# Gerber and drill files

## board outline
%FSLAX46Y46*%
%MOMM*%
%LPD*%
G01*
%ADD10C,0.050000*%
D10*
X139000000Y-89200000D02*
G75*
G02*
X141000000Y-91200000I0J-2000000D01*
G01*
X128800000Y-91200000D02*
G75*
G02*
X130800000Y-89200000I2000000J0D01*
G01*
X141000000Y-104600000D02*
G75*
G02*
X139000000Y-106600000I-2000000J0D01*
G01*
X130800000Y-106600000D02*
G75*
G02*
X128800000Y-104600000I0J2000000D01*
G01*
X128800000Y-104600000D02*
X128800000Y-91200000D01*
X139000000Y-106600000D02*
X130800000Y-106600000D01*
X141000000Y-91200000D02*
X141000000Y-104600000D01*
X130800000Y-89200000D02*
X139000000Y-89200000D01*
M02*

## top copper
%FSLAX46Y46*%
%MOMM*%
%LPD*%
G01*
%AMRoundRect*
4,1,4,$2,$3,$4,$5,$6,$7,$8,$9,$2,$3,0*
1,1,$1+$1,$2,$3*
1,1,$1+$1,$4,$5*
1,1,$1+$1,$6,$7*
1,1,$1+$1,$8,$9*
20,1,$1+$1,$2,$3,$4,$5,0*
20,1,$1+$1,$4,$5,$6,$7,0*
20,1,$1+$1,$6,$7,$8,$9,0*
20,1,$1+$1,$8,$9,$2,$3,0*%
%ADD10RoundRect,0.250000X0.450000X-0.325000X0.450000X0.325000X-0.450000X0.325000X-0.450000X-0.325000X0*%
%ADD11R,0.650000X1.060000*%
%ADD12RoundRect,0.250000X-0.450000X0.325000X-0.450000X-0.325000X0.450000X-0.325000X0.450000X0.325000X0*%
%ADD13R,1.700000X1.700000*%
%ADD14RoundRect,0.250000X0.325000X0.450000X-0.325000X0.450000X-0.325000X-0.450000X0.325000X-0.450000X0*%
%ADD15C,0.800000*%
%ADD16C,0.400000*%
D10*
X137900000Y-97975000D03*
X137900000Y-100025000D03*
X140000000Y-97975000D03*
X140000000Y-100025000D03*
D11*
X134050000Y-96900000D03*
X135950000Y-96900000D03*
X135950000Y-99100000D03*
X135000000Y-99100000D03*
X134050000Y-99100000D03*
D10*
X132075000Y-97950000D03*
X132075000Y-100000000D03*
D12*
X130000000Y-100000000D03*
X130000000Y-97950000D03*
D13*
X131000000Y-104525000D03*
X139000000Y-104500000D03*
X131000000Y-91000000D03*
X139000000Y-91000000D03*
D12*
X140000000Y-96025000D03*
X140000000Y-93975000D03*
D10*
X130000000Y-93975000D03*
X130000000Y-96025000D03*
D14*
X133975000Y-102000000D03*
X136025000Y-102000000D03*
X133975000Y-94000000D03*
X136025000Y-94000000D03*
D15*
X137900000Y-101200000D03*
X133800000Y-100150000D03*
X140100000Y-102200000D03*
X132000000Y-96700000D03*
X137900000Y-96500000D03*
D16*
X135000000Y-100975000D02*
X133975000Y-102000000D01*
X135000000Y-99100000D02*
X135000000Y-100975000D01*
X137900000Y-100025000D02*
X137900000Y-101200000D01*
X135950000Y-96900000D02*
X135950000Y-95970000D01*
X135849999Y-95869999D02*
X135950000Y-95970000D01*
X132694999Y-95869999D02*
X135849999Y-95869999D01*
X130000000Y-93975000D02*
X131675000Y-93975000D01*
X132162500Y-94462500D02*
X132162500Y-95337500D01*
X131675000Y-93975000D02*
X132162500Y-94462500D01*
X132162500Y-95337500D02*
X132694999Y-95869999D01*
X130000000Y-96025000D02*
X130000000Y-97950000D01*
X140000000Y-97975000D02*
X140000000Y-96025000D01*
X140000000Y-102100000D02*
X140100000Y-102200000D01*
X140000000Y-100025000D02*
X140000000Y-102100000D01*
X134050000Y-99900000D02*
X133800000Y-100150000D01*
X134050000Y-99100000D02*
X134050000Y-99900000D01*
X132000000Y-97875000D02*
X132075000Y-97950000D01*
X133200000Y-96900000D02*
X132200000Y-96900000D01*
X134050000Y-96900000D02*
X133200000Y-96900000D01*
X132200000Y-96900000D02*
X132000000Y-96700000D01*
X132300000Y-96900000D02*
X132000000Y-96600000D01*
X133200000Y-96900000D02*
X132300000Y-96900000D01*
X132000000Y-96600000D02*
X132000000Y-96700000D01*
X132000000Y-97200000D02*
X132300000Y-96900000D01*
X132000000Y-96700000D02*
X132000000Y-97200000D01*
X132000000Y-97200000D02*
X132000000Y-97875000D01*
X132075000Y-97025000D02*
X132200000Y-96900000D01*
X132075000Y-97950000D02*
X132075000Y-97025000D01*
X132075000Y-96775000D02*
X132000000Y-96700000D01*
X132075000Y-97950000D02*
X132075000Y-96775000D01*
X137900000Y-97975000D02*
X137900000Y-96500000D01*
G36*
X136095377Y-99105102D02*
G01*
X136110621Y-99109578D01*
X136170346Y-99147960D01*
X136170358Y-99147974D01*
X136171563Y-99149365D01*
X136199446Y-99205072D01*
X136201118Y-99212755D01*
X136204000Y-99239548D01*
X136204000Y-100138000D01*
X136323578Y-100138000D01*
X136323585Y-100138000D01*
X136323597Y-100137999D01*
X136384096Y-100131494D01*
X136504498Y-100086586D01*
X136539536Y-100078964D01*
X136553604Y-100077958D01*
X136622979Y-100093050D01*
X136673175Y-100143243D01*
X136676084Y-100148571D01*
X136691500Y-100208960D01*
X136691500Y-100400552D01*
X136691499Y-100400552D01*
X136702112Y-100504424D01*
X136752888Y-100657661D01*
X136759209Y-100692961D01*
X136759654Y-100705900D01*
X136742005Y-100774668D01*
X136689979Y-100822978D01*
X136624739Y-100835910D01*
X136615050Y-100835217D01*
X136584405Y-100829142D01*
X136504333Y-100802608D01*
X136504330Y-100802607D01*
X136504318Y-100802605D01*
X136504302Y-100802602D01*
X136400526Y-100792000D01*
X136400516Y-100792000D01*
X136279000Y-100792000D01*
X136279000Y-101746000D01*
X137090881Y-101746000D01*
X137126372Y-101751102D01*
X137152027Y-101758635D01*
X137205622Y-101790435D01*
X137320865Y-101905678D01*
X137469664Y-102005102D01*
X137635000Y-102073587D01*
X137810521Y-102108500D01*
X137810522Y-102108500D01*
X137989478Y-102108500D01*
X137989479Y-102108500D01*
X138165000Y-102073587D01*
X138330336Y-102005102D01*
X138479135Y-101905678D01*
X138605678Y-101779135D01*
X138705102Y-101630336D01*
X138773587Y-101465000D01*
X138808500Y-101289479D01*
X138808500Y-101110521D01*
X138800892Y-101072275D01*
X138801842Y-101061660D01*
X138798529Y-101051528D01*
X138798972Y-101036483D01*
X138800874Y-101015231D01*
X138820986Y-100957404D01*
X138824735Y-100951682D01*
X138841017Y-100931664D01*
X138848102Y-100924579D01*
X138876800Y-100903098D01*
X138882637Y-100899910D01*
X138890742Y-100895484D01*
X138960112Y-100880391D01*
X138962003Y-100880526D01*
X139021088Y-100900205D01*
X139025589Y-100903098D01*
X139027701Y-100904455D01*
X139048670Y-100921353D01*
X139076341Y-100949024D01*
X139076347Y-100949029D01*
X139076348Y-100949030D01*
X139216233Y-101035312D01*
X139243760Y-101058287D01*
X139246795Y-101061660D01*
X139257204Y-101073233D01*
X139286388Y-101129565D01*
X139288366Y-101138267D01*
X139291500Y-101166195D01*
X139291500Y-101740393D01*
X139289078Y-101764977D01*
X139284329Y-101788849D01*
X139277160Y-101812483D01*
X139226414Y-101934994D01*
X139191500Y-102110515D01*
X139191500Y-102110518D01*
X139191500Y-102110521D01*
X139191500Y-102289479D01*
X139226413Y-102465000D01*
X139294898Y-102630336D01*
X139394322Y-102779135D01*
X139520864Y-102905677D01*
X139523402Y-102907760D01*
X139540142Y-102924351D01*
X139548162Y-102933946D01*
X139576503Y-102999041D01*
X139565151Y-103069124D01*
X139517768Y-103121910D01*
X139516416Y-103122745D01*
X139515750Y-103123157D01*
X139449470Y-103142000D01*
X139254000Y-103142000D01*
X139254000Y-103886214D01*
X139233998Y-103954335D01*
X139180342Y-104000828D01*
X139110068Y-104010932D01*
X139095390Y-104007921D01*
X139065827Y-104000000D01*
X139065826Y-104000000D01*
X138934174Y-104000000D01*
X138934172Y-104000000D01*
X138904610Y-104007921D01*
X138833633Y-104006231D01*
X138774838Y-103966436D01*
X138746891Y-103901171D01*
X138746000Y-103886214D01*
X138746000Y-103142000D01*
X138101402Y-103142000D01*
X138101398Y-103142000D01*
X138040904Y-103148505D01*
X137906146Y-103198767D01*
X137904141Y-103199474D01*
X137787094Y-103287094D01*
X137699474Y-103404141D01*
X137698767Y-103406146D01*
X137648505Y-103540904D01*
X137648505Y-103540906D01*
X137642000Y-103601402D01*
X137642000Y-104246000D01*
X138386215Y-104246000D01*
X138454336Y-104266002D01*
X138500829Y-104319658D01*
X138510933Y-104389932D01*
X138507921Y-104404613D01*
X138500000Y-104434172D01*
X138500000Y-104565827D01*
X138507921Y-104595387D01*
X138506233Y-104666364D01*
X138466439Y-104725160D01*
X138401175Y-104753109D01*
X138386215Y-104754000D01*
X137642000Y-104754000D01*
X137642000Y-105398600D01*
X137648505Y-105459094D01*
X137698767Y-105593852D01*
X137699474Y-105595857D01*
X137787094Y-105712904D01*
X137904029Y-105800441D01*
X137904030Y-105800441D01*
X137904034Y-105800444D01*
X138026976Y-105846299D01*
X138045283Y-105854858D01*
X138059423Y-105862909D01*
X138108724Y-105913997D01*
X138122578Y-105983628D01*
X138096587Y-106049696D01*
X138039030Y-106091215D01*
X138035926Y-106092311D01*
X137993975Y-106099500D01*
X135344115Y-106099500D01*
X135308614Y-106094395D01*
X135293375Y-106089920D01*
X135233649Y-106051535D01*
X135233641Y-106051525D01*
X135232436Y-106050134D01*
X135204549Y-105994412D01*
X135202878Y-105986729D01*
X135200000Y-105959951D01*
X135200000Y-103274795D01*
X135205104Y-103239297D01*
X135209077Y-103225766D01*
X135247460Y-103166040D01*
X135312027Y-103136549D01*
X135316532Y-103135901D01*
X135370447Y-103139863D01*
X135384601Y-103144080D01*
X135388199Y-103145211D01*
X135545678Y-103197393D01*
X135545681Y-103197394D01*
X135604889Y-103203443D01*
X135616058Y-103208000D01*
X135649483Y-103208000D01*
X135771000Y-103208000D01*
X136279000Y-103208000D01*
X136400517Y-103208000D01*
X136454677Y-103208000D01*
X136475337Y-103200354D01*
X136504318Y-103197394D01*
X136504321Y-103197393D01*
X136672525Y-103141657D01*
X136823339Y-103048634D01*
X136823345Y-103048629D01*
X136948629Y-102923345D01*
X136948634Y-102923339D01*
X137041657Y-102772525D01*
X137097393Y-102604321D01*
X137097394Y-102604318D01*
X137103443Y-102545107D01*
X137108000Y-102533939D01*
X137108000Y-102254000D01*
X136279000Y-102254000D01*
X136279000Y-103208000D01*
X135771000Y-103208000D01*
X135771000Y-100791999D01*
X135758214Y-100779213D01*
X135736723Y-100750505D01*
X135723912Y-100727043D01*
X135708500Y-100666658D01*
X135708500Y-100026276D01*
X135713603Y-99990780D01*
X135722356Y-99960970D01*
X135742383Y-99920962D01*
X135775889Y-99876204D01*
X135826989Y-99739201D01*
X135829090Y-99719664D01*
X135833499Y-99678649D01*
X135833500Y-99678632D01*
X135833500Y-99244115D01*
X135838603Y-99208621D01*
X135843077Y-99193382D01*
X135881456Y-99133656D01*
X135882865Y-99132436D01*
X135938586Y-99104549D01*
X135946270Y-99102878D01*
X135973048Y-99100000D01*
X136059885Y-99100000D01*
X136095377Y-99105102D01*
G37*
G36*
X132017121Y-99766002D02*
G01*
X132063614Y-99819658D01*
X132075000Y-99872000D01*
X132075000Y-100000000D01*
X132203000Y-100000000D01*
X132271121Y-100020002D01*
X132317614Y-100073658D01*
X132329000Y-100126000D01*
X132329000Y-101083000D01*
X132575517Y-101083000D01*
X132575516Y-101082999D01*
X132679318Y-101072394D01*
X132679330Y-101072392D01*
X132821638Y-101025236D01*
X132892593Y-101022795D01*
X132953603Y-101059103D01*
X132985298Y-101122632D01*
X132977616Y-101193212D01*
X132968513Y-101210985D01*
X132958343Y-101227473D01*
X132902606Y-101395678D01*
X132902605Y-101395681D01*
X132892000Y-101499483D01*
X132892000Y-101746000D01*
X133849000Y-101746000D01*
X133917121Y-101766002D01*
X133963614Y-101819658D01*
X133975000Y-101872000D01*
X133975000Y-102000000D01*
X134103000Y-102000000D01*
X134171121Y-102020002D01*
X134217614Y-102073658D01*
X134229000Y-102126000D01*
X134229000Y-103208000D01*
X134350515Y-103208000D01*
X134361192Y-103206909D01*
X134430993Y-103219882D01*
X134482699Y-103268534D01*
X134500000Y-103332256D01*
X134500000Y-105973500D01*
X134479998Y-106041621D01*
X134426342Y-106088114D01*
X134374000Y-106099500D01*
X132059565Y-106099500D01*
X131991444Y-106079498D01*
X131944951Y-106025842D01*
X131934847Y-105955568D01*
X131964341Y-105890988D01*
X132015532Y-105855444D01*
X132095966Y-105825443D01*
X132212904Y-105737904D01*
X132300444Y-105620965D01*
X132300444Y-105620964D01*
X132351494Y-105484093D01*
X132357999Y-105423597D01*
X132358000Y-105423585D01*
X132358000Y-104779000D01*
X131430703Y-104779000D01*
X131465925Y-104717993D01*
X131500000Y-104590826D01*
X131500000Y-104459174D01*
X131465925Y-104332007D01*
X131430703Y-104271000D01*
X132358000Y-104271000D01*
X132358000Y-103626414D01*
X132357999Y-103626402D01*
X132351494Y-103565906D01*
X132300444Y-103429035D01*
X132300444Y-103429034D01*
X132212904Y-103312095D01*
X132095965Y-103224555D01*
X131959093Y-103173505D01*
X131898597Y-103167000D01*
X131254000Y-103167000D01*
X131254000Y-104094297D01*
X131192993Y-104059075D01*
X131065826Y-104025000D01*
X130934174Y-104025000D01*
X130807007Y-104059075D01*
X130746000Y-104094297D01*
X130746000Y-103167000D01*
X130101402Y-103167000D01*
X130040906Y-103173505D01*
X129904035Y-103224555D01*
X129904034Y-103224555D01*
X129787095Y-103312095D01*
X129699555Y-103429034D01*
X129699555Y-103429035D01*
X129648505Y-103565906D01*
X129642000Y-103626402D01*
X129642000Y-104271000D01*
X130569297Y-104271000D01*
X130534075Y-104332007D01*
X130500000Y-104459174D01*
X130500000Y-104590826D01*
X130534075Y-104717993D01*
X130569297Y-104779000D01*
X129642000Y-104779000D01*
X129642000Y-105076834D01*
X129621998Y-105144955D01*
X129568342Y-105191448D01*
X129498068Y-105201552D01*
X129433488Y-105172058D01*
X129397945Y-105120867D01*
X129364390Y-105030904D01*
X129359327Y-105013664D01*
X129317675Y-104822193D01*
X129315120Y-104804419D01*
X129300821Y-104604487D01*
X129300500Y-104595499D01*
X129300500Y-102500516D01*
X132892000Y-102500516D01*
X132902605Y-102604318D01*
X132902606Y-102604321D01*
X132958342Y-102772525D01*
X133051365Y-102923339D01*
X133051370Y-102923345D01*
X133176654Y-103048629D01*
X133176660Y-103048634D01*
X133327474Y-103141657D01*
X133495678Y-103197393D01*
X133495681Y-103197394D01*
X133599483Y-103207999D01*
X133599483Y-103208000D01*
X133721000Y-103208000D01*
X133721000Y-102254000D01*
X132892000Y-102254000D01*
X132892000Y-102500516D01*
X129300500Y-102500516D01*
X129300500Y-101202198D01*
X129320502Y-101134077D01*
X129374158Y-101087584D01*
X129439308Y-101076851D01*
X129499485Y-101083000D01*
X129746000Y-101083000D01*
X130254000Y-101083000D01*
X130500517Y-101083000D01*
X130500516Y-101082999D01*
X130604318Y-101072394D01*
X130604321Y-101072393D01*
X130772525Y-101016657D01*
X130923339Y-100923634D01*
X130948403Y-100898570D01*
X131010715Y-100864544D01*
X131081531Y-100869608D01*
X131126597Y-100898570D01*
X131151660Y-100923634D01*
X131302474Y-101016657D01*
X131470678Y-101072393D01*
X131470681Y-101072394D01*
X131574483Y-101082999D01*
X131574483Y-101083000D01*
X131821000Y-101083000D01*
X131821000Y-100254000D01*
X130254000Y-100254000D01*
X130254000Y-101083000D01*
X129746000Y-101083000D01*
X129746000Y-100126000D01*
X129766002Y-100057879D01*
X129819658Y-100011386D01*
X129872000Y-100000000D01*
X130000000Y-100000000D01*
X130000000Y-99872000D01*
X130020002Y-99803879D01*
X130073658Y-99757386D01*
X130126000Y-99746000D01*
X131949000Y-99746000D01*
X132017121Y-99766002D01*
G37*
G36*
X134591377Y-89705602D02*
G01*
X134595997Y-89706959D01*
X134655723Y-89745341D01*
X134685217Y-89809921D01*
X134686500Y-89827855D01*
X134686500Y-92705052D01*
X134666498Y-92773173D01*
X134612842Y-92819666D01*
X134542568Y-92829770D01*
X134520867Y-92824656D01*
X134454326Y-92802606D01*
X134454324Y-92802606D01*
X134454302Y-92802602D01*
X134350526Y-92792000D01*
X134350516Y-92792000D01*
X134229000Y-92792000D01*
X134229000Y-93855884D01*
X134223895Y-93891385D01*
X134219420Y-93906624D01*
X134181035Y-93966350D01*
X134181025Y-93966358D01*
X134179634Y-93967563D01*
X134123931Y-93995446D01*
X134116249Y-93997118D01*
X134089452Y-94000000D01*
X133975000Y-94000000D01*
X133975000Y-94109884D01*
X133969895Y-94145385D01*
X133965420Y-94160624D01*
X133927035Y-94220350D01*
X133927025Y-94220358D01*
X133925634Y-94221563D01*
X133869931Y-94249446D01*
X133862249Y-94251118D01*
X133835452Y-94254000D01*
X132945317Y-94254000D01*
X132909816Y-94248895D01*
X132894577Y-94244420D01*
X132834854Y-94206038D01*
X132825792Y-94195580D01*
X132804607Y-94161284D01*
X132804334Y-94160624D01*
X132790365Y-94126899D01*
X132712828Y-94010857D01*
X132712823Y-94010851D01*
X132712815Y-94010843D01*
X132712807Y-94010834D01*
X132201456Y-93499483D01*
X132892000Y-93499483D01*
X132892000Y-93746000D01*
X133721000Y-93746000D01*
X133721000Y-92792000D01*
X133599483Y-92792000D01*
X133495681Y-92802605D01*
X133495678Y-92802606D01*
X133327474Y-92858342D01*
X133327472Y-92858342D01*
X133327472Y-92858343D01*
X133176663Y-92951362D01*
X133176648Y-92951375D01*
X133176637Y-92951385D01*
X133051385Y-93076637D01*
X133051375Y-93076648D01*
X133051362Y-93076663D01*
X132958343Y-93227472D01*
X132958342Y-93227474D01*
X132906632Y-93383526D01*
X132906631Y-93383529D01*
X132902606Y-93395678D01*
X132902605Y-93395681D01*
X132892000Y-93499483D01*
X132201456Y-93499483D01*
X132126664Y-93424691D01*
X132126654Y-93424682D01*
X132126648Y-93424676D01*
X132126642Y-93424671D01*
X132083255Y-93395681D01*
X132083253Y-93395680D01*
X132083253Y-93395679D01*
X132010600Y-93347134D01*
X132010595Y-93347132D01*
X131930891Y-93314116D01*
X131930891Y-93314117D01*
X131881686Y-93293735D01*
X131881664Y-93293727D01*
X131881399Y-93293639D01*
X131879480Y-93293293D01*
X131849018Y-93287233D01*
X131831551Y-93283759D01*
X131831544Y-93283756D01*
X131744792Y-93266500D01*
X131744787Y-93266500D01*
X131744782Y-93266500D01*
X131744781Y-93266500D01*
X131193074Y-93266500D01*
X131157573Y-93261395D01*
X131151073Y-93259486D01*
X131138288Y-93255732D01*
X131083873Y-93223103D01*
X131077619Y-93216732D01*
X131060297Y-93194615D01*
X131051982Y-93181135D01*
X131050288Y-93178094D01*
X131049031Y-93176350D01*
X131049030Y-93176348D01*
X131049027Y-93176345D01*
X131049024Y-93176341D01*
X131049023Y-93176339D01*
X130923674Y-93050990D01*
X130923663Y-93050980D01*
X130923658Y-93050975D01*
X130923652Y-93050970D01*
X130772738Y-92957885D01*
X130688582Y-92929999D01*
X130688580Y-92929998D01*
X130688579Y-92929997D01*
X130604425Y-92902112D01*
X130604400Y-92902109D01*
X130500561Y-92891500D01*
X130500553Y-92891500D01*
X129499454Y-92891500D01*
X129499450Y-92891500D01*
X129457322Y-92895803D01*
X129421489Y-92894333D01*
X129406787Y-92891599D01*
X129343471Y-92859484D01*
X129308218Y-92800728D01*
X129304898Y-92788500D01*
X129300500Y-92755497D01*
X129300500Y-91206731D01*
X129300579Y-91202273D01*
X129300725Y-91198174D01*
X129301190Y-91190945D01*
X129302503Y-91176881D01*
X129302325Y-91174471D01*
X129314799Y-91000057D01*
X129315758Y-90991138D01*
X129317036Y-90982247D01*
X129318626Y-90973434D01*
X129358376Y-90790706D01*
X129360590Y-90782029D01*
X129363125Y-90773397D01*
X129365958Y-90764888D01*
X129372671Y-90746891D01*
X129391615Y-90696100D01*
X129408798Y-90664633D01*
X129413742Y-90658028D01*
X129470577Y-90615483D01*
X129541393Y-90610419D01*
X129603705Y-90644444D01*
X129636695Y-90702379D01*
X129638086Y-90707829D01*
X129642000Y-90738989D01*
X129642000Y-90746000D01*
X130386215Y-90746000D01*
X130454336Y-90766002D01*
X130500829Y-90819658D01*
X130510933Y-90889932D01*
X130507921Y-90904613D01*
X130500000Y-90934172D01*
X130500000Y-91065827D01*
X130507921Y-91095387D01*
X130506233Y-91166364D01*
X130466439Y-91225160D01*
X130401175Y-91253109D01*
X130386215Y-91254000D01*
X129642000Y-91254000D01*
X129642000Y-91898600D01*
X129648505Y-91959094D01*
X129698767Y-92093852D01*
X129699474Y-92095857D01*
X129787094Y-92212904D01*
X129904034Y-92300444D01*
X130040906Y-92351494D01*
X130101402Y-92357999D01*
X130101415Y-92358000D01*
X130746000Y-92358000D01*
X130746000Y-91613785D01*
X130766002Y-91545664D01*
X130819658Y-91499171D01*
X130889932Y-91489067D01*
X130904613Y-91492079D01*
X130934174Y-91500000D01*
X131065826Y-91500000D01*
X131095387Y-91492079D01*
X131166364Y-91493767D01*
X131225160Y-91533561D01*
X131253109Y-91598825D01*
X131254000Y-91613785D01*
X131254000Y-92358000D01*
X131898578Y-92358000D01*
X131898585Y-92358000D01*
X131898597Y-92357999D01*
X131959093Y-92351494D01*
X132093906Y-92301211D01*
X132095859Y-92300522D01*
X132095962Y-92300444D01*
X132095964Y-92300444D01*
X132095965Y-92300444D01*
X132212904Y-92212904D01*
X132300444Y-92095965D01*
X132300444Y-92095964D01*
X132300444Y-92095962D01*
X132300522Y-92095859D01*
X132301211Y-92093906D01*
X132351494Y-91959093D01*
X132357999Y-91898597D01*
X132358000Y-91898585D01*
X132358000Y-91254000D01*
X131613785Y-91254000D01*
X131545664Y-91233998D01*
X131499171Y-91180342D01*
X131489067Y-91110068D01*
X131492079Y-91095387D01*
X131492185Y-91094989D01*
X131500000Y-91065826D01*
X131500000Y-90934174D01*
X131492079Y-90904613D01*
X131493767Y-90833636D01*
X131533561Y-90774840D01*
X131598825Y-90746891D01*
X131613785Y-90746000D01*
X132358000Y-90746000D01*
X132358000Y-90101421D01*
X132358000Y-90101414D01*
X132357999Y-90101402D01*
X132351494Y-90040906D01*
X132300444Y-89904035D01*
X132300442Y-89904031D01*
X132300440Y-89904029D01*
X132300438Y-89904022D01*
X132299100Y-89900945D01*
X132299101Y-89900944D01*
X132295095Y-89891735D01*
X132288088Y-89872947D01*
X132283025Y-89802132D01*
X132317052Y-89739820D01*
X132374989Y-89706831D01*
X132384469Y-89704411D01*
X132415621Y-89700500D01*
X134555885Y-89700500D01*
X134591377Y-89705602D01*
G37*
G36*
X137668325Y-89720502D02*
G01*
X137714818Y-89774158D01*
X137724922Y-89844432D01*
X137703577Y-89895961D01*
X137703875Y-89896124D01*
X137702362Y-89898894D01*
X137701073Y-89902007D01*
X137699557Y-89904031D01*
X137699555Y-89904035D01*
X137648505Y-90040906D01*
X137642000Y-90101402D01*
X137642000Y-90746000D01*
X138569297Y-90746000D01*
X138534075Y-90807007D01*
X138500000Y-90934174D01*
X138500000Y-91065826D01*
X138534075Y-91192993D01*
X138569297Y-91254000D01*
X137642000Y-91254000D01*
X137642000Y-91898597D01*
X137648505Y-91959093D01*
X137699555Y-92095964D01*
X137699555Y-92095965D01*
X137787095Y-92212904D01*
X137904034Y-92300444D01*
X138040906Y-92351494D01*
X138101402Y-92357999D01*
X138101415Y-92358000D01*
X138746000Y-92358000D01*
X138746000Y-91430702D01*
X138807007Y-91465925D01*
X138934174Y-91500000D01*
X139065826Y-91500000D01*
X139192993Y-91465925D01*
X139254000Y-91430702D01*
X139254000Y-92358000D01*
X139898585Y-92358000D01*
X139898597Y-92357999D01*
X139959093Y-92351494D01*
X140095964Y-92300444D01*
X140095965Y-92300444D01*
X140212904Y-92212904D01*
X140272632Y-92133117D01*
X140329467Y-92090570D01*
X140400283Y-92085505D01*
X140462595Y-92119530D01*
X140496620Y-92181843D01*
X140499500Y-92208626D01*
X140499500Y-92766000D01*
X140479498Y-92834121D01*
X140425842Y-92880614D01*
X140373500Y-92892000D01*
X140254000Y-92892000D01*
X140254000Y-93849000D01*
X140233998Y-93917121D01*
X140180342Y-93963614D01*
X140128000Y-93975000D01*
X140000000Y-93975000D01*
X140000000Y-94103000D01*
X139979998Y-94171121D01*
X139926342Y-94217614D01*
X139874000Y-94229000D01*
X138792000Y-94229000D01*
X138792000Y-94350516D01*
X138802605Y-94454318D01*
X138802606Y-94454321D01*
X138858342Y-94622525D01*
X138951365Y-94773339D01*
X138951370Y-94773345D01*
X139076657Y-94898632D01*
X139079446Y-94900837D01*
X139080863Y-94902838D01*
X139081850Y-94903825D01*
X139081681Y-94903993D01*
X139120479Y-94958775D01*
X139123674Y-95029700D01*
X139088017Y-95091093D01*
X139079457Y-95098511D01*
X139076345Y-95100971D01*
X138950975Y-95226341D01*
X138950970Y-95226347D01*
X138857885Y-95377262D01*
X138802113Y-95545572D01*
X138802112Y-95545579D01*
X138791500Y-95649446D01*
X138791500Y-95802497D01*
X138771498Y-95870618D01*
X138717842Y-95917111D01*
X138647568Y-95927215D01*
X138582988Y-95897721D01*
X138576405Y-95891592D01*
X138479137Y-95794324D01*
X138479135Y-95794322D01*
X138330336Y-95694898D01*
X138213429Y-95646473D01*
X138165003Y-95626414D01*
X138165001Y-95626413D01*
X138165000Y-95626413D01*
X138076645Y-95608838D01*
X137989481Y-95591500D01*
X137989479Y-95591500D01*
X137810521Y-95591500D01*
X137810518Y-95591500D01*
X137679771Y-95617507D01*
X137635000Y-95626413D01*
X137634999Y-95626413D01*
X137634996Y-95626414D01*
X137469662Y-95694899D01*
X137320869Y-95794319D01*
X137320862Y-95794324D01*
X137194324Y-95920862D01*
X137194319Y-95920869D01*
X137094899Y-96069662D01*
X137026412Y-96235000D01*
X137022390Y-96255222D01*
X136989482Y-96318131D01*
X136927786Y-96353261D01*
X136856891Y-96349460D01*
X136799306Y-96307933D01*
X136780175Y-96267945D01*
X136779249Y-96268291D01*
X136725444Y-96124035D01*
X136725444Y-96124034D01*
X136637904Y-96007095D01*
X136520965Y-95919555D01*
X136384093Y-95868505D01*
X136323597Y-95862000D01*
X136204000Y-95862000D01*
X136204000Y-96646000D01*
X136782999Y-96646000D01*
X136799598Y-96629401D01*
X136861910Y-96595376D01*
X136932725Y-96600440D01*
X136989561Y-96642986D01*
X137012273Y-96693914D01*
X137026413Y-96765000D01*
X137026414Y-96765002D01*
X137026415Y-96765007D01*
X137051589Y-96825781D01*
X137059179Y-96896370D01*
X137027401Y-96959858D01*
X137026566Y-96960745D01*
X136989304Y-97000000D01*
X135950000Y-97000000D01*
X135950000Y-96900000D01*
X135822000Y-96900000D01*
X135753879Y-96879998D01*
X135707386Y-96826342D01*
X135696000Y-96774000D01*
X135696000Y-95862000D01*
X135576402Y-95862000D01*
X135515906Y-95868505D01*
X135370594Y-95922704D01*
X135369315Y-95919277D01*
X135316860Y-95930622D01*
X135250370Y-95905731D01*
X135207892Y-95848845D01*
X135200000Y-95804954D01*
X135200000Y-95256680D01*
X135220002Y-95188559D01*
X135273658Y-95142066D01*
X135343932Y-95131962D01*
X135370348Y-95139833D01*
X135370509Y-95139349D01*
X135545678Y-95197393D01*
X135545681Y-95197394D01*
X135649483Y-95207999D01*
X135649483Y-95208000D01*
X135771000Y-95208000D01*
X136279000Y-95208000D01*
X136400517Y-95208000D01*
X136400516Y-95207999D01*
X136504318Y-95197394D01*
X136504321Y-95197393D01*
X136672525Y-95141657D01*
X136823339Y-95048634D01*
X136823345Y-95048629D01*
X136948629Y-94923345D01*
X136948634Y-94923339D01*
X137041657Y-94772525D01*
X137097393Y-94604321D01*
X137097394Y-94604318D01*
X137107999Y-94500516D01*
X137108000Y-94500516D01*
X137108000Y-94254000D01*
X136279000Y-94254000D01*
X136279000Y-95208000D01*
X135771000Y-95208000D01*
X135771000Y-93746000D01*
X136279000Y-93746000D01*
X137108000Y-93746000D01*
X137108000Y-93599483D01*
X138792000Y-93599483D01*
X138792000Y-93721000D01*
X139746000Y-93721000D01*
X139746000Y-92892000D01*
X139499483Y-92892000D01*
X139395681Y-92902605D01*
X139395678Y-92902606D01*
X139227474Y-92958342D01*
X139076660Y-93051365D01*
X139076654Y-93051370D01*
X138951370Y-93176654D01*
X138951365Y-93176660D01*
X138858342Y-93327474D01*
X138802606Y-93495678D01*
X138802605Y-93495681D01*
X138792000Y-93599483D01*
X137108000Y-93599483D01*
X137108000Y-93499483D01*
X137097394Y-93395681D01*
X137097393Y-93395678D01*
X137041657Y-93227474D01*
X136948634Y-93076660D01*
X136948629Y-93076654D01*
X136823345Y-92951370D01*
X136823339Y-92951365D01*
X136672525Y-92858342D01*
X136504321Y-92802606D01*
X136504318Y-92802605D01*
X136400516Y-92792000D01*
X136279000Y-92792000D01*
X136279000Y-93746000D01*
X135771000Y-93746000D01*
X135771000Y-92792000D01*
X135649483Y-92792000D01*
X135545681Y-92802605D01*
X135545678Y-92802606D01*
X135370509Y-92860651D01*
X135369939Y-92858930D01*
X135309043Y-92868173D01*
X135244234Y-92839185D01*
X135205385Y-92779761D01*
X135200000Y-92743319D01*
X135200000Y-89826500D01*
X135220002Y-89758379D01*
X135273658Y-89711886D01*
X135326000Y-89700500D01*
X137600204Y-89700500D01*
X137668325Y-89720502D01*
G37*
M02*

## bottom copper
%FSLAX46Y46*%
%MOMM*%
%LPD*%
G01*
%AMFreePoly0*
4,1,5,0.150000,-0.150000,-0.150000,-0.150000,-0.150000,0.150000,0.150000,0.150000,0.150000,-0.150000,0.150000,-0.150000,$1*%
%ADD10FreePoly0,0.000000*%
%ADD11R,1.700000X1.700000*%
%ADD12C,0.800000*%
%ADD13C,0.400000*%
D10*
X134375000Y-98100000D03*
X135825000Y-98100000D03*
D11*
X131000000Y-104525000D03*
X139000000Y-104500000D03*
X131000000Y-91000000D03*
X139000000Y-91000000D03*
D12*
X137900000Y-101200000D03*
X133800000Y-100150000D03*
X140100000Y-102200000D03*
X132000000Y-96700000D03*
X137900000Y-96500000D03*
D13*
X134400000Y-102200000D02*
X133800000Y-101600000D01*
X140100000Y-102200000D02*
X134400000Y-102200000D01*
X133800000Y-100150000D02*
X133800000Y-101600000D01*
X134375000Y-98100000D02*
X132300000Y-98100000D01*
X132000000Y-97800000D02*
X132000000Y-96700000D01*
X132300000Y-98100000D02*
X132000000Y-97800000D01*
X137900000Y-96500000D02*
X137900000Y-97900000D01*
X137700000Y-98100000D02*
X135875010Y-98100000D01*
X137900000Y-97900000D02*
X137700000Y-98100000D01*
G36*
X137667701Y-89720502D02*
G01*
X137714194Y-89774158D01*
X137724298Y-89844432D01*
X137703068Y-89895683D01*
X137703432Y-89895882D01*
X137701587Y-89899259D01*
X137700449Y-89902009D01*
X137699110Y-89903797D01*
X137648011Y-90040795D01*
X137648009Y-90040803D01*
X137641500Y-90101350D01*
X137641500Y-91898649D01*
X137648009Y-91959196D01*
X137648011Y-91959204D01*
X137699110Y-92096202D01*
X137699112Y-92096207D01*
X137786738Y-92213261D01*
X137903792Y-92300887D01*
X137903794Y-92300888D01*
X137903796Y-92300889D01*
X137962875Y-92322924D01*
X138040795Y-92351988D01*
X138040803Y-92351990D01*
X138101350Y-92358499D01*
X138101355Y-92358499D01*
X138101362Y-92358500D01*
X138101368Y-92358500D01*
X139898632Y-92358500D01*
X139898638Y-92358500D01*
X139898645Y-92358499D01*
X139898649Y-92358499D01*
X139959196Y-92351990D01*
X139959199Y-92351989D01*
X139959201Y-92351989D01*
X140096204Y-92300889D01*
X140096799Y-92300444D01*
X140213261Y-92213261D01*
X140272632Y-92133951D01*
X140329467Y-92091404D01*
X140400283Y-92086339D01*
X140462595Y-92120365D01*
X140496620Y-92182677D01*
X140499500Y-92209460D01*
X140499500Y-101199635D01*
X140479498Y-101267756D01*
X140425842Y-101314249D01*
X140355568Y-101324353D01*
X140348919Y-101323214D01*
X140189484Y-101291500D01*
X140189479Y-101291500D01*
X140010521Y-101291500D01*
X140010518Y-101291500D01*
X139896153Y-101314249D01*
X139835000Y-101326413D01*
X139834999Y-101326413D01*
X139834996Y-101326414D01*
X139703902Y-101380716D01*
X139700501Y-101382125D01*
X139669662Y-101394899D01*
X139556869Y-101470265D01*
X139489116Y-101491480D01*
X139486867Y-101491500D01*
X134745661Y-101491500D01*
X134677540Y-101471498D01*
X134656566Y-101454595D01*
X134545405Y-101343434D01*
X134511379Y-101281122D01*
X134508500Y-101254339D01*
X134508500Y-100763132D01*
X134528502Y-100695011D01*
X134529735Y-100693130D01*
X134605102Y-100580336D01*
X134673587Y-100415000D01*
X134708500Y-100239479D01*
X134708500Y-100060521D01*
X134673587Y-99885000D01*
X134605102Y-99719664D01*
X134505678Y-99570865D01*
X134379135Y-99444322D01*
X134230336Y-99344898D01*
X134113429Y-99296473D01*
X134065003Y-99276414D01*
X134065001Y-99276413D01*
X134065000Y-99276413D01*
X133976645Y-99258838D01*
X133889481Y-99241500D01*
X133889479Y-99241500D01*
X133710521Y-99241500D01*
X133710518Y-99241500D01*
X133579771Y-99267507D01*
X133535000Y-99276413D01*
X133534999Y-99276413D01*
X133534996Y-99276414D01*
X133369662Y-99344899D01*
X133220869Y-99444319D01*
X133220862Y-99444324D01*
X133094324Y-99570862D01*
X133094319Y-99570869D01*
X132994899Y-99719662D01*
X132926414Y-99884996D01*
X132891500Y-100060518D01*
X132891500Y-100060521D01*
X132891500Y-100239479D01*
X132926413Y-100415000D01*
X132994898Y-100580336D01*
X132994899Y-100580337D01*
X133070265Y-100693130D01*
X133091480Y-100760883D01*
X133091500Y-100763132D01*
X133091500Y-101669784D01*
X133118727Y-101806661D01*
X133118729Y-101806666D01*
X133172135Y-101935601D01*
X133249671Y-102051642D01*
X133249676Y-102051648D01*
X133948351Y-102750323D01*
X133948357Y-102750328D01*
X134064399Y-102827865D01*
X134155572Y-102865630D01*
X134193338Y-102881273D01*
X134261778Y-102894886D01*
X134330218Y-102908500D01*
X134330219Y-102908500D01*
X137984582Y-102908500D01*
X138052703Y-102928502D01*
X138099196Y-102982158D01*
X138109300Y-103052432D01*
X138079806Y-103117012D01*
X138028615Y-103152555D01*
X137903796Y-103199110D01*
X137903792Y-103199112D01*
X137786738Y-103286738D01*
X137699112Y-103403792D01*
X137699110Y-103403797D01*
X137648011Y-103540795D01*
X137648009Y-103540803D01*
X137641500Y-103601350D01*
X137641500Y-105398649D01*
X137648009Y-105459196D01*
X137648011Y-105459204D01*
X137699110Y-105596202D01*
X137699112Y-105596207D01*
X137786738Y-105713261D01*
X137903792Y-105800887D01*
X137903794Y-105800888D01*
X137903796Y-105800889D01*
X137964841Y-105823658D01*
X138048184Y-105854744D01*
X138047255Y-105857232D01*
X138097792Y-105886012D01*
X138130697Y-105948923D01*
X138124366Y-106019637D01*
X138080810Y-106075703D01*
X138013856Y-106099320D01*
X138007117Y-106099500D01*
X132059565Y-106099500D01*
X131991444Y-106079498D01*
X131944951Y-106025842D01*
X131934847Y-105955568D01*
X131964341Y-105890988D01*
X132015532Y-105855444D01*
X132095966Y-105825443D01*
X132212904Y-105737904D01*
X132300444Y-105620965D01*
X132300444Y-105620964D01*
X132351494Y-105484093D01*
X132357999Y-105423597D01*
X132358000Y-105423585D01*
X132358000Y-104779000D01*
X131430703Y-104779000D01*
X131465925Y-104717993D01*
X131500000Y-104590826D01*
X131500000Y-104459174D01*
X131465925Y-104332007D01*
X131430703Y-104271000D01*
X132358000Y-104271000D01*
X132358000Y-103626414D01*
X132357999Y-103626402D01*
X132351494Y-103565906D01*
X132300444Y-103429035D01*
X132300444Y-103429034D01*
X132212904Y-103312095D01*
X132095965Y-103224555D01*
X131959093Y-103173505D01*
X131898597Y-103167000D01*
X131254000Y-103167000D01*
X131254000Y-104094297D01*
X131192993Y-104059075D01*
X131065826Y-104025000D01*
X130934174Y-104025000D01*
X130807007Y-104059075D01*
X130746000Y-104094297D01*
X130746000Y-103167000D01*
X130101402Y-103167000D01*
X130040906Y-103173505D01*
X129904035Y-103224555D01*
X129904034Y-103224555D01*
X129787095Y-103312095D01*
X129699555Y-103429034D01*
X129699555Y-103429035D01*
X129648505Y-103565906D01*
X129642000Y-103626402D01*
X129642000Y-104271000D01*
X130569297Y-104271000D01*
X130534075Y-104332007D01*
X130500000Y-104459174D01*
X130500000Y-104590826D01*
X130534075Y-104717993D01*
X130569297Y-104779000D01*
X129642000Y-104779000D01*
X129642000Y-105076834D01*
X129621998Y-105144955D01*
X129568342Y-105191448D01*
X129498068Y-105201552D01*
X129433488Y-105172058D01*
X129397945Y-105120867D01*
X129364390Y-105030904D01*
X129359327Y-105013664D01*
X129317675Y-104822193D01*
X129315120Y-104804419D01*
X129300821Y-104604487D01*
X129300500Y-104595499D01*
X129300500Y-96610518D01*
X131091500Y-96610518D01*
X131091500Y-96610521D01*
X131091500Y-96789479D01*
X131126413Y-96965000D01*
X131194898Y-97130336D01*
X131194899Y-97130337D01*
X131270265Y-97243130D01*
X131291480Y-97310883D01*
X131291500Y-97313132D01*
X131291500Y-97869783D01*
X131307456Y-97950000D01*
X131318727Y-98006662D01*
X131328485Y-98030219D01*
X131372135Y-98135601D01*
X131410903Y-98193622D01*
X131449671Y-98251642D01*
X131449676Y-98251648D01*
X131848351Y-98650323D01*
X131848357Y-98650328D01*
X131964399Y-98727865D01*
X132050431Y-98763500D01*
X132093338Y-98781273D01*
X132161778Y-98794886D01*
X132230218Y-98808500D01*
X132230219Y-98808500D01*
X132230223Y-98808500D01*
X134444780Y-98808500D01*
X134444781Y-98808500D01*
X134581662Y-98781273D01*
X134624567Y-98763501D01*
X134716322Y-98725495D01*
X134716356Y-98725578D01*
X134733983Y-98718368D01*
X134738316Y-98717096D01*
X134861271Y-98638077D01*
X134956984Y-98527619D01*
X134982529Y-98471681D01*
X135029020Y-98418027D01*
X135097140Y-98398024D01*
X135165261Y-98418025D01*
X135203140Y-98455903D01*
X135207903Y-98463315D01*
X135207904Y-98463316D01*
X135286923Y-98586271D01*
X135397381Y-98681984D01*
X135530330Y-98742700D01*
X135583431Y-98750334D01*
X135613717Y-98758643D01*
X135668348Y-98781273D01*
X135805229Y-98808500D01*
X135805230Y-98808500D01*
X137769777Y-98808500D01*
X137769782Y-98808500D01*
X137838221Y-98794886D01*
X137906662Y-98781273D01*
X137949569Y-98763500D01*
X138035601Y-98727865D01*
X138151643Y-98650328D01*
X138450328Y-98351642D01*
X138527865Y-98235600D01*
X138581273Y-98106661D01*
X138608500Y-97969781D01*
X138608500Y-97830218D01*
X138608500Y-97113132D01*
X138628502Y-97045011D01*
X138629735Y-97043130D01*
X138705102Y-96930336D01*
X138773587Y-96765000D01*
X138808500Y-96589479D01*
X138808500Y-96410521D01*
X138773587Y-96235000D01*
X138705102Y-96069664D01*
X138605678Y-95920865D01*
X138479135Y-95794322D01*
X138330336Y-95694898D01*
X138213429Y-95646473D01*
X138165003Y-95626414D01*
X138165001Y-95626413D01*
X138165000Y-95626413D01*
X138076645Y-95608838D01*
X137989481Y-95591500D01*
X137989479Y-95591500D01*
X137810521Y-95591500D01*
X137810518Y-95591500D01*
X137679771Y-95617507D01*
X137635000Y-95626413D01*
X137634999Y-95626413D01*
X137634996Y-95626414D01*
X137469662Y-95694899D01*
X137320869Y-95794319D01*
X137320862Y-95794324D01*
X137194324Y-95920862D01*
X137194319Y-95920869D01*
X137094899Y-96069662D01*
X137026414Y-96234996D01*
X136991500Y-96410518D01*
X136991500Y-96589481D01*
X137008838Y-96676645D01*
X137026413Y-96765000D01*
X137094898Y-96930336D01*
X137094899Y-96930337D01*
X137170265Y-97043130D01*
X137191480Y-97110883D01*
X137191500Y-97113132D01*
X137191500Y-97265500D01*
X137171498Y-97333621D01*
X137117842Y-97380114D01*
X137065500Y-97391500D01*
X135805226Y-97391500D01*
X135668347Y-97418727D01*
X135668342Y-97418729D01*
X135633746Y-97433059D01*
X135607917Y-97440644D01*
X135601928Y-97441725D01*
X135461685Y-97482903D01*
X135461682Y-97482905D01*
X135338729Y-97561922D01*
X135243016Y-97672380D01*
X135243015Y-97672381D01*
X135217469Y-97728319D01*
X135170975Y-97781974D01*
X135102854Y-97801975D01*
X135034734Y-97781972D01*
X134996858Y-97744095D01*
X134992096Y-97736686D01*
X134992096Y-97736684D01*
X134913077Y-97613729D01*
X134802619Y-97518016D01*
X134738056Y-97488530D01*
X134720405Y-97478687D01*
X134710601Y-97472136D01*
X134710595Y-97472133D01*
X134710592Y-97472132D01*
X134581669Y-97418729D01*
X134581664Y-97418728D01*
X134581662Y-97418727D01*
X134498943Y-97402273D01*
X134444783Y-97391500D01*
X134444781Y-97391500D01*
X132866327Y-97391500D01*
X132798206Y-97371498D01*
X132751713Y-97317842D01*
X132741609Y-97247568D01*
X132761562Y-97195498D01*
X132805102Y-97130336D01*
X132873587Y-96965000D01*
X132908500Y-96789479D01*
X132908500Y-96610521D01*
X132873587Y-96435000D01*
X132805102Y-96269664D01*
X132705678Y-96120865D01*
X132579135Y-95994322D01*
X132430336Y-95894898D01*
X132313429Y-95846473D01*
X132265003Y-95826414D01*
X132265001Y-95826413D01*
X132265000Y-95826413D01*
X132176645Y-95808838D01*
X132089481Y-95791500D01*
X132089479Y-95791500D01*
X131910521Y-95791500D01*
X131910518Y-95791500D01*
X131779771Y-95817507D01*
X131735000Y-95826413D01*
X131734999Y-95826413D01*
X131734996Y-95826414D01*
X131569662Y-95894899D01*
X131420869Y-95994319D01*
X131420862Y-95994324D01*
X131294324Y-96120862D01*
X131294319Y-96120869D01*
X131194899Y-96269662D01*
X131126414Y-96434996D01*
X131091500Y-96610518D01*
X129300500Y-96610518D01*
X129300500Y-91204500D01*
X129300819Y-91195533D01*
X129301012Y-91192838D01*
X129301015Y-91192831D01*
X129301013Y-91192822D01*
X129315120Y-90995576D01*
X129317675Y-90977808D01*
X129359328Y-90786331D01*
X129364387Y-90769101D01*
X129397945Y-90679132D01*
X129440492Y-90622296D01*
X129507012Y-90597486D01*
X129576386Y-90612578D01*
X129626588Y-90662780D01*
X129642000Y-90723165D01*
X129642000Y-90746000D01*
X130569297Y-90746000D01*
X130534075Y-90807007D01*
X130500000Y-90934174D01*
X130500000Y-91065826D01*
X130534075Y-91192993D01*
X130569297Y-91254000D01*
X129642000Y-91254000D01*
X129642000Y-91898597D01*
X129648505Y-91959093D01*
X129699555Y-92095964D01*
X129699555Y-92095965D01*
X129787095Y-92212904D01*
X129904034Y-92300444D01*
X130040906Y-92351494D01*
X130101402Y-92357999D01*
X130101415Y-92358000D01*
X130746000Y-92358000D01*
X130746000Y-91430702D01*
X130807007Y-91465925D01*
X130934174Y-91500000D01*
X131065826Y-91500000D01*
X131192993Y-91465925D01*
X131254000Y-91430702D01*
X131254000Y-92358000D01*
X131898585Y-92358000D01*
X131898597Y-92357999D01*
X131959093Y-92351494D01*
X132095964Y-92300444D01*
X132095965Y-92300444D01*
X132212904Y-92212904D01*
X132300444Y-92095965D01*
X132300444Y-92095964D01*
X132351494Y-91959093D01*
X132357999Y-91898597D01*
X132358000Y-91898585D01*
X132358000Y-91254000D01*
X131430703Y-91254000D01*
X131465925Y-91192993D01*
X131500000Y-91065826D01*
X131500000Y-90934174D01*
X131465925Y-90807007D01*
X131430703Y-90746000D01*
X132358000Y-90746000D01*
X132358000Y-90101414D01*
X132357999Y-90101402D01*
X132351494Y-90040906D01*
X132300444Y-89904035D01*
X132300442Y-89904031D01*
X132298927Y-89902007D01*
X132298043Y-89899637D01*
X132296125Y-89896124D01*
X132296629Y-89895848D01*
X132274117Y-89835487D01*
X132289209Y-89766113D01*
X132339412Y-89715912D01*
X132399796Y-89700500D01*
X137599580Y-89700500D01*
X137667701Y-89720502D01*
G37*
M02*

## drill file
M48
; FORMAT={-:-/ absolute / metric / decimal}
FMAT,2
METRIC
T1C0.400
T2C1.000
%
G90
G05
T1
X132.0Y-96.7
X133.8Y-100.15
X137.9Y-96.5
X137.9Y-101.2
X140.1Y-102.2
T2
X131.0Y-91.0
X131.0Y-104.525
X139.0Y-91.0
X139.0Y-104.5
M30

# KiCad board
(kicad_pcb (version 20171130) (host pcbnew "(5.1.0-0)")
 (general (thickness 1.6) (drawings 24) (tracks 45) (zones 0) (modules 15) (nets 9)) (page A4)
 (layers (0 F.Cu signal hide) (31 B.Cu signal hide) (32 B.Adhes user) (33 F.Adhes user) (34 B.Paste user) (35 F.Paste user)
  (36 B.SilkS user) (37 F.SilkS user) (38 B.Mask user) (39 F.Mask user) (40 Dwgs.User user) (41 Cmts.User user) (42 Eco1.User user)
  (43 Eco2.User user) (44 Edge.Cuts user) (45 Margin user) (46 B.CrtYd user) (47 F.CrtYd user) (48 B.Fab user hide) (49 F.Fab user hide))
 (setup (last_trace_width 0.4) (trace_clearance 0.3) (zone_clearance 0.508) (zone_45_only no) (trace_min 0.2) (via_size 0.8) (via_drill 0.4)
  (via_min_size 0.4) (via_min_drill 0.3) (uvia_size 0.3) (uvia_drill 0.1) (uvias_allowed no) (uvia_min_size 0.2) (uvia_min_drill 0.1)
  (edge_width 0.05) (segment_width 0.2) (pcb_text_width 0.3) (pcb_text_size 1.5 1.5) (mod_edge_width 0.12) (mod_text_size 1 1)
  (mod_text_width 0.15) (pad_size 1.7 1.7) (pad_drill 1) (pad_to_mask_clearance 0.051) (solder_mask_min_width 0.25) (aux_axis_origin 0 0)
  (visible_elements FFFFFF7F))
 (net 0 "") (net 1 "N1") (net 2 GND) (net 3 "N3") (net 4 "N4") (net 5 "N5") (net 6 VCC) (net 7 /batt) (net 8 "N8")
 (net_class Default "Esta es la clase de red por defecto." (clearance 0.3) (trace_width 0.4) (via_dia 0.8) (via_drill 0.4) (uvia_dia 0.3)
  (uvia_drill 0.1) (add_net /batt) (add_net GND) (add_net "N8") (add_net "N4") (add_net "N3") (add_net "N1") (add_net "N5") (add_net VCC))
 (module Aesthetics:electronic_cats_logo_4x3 (layer B.Cu) (at 135 94.1 180)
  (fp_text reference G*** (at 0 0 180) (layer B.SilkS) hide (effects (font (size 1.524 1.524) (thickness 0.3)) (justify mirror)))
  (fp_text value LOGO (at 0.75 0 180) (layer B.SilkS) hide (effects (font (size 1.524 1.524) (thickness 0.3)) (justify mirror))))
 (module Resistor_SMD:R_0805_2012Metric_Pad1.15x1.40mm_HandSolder (layer F.Cu) (at 137.9 99 90)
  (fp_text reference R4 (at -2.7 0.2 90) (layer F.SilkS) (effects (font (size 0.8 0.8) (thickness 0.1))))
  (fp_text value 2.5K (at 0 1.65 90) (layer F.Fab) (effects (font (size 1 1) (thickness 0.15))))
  (pad 2 smd roundrect (at 1.025 0 90) (size 1.15 1.4) (layers F.Cu F.Paste F.Mask) (roundrect_rratio 0.217391) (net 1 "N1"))
  (pad 1 smd roundrect (at -1.025 0 90) (size 1.15 1.4) (layers F.Cu F.Paste F.Mask) (roundrect_rratio 0.217391) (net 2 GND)))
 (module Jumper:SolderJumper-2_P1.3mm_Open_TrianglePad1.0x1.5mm (layer B.Cu) (at 135.1 98.1)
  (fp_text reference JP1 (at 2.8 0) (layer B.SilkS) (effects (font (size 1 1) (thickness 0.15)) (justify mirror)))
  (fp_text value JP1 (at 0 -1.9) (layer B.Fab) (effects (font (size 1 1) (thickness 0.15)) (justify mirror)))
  (pad 1 smd custom (at -0.725 0) (size 0.3 0.3) (layers B.Cu B.Mask) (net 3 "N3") (zone_connect 2)
   (options (clearance outline) (anchor rect)) (primitives))
  (pad 2 smd custom (at 0.725 0) (size 0.3 0.3) (layers B.Cu B.Mask) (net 1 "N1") (zone_connect 2)
   (options (clearance outline) (anchor rect)) (primitives)))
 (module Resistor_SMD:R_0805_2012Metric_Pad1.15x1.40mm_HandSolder (layer F.Cu) (at 140 99 90)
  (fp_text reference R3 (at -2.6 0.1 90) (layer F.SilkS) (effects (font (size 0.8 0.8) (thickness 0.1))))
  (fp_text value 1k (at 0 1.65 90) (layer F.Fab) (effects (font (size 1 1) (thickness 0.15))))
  (pad 2 smd roundrect (at 1.025 0 90) (size 1.15 1.4) (layers F.Cu F.Paste F.Mask) (roundrect_rratio 0.217391) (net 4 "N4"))
  (pad 1 smd roundrect (at -1.025 0 90) (size 1.15 1.4) (layers F.Cu F.Paste F.Mask) (roundrect_rratio 0.217391) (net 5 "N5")))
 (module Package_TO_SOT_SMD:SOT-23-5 (layer F.Cu) (at 135 98 90)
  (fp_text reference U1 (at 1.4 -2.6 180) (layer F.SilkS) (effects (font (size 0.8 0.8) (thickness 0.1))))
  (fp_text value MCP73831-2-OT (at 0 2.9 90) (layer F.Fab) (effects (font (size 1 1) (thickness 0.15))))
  (pad 5 smd rect (at 1.1 -0.95 90) (size 1.06 0.65) (layers F.Cu F.Paste F.Mask) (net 3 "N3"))
  (pad 4 smd rect (at 1.1 0.95 90) (size 1.06 0.65) (layers F.Cu F.Paste F.Mask) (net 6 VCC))
  (pad 3 smd rect (at -1.1 0.95 90) (size 1.06 0.65) (layers F.Cu F.Paste F.Mask) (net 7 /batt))
  (pad 2 smd rect (at -1.1 0 90) (size 1.06 0.65) (layers F.Cu F.Paste F.Mask) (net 2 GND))
  (pad 1 smd rect (at -1.1 -0.95 90) (size 1.06 0.65) (layers F.Cu F.Paste F.Mask) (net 5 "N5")))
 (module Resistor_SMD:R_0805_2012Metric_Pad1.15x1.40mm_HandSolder (layer F.Cu) (at 132.075 98.975 90)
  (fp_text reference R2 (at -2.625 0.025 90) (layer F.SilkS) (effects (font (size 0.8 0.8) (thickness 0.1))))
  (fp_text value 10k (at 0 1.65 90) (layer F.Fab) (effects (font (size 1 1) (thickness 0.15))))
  (pad 2 smd roundrect (at 1.025 0 90) (size 1.15 1.4) (layers F.Cu F.Paste F.Mask) (roundrect_rratio 0.217391) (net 3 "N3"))
  (pad 1 smd roundrect (at -1.025 0 90) (size 1.15 1.4) (layers F.Cu F.Paste F.Mask) (roundrect_rratio 0.217391) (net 2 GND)))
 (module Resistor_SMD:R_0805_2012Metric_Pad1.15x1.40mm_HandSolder (layer F.Cu) (at 130 98.975 270)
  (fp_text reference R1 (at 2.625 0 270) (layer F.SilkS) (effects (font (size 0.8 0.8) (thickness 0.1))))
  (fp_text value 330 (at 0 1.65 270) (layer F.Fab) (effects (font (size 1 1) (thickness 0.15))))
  (pad 2 smd roundrect (at 1.025 0 270) (size 1.15 1.4) (layers F.Cu F.Paste F.Mask) (roundrect_rratio 0.217391) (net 2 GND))
  (pad 1 smd roundrect (at -1.025 0 270) (size 1.15 1.4) (layers F.Cu F.Paste F.Mask) (roundrect_rratio 0.217391) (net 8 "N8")))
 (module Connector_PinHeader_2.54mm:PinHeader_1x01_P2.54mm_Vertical (layer B.Cu) (at 131 104.5)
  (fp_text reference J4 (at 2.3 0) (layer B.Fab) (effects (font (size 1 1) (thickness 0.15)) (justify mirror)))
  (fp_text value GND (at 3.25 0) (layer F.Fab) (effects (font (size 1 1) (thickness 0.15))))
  (pad 1 thru_hole rect (at 0 0.025) (size 1.7 1.7) (drill 1) (layers *.Cu *.Mask) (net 2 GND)))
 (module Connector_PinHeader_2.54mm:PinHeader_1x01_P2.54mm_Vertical (layer B.Cu) (at 139 104.5)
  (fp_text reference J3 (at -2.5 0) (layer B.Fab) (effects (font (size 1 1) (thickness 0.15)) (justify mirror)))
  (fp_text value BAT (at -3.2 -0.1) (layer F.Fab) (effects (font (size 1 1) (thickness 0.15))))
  (pad 1 thru_hole rect (at 0 0) (size 1.7 1.7) (drill 1) (layers *.Cu *.Mask) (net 7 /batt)))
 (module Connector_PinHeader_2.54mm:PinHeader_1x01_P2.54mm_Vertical (layer B.Cu) (at 131 91)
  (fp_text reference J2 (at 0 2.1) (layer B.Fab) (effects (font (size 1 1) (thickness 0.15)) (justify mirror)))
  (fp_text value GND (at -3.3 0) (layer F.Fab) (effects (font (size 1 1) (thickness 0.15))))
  (pad 1 thru_hole rect (at 0 0) (size 1.7 1.7) (drill 1) (layers *.Cu *.Mask) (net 2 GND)))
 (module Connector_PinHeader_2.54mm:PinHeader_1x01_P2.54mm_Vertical (layer B.Cu) (at 139 91)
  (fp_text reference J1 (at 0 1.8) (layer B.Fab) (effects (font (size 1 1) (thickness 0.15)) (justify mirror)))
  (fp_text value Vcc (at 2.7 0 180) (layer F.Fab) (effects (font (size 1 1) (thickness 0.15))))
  (pad 1 thru_hole rect (at 0 0) (size 1.7 1.7) (drill 1) (layers *.Cu *.Mask) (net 6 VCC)))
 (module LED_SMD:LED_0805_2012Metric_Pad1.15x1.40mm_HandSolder (layer F.Cu) (at 140 95 270)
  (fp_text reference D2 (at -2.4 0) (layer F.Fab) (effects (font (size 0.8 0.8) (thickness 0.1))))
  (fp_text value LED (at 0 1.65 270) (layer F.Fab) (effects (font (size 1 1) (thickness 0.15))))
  (pad 2 smd roundrect (at 1.025 0 270) (size 1.15 1.4) (layers F.Cu F.Paste F.Mask) (roundrect_rratio 0.217391) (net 4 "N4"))
  (pad 1 smd roundrect (at -1.025 0 270) (size 1.15 1.4) (layers F.Cu F.Paste F.Mask) (roundrect_rratio 0.217391) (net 6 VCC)))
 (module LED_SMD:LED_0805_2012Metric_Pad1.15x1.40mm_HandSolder (layer F.Cu) (at 130 95 90)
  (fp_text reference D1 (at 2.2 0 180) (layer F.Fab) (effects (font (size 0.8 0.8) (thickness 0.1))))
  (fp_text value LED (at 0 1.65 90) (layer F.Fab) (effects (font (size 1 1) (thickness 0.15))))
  (pad 2 smd roundrect (at 1.025 0 90) (size 1.15 1.4) (layers F.Cu F.Paste F.Mask) (roundrect_rratio 0.217391) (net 6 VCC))
  (pad 1 smd roundrect (at -1.025 0 90) (size 1.15 1.4) (layers F.Cu F.Paste F.Mask) (roundrect_rratio 0.217391) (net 8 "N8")))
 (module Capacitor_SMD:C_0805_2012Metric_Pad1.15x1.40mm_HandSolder (layer F.Cu) (at 135 102 180)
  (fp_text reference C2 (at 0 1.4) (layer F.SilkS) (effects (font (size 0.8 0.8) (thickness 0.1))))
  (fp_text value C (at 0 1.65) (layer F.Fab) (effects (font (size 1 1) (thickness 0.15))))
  (pad 2 smd roundrect (at 1.025 0 180) (size 1.15 1.4) (layers F.Cu F.Paste F.Mask) (roundrect_rratio 0.217391) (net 2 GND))
  (pad 1 smd roundrect (at -1.025 0 180) (size 1.15 1.4) (layers F.Cu F.Paste F.Mask) (roundrect_rratio 0.217391) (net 7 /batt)))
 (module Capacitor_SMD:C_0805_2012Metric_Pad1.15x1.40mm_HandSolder (layer F.Cu) (at 135 94 180)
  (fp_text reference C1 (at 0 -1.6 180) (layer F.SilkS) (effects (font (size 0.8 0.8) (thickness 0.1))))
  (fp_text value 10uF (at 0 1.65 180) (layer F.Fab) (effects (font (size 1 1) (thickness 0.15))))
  (pad 2 smd roundrect (at 1.025 0 180) (size 1.15 1.4) (layers F.Cu F.Paste F.Mask) (roundrect_rratio 0.217391) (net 2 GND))
  (pad 1 smd roundrect (at -1.025 0 180) (size 1.15 1.4) (layers F.Cu F.Paste F.Mask) (roundrect_rratio 0.217391) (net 6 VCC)))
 (gr_arc (start 139 91.2) (end 141 91.2) (angle -90) (layer Edge.Cuts) (width 0.05))
 (gr_arc (start 130.8 91.2) (end 130.8 89.2) (angle -90) (layer Edge.Cuts) (width 0.05))
 (gr_arc (start 139 104.6) (end 139 106.6) (angle -90) (layer Edge.Cuts) (width 0.05))
 (gr_arc (start 130.8 104.6) (end 128.8 104.6) (angle -90) (layer Edge.Cuts) (width 0.05))
 (gr_line (start 128.8 104.6) (end 128.8 91.2) (layer Edge.Cuts) (width 0.05))
 (gr_line (start 139 106.6) (end 130.8 106.6) (layer Edge.Cuts) (width 0.05))
 (gr_line (start 141 91.2) (end 141 104.6) (layer Edge.Cuts) (width 0.05))
 (gr_line (start 130.8 89.2) (end 139 89.2) (layer Edge.Cuts) (width 0.05))
 (segment (start 135 100.975) (end 133.975 102) (width 0.4) (layer F.Cu) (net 2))
 (segment (start 135 99.1) (end 135 100.975) (width 0.4) (layer F.Cu) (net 2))
 (via (at 137.9 101.2) (size 0.8) (drill 0.4) (layers F.Cu B.Cu) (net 2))
 (segment (start 137.9 100.025) (end 137.9 101.2) (width 0.4) (layer F.Cu) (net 2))
 (segment (start 135.95 96.9) (end 135.95 95.97) (width 0.4) (layer F.Cu) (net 6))
 (segment (start 135.849999 95.869999) (end 135.95 95.97) (width 0.4) (layer F.Cu) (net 6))
 (segment (start 132.694999 95.869999) (end 135.849999 95.869999) (width 0.4) (layer F.Cu) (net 6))
 (segment (start 130 93.975) (end 131.675 93.975) (width 0.4) (layer F.Cu) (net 6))
 (segment (start 132.1625 94.4625) (end 132.1625 95.3375) (width 0.4) (layer F.Cu) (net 6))
 (segment (start 131.675 93.975) (end 132.1625 94.4625) (width 0.4) (layer F.Cu) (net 6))
 (segment (start 132.1625 95.3375) (end 132.694999 95.869999) (width 0.4) (layer F.Cu) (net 6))
 (segment (start 130 96.025) (end 130 97.95) (width 0.4) (layer F.Cu) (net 8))
 (segment (start 140 97.975) (end 140 96.025) (width 0.4) (layer F.Cu) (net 4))
 (segment (start 140 102.1) (end 140.1 102.2) (width 0.4) (layer F.Cu) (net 5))
 (segment (start 140 100.025) (end 140 102.1) (width 0.4) (layer F.Cu) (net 5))
 (via (at 133.8 100.15) (size 0.8) (drill 0.4) (layers F.Cu B.Cu) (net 5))
 (via (at 140.1 102.2) (size 0.8) (drill 0.4) (layers F.Cu B.Cu) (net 5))
 (segment (start 134.05 99.9) (end 133.8 100.15) (width 0.4) (layer F.Cu) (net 5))
 (segment (start 134.05 99.1) (end 134.05 99.9) (width 0.4) (layer F.Cu) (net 5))
 (segment (start 134.4 102.2) (end 133.8 101.6) (width 0.4) (layer B.Cu) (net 5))
 (segment (start 140.1 102.2) (end 134.4 102.2) (width 0.4) (layer B.Cu) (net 5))
 (segment (start 133.8 100.15) (end 133.8 101.6) (width 0.4) (layer B.Cu) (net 5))
 (segment (start 132 97.875) (end 132.075 97.95) (width 0.4) (layer F.Cu) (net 3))
 (segment (start 133.2 96.9) (end 132.2 96.9) (width 0.4) (layer F.Cu) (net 3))
 (segment (start 134.05 96.9) (end 133.2 96.9) (width 0.4) (layer F.Cu) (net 3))
 (segment (start 132.2 96.9) (end 132 96.7) (width 0.4) (layer F.Cu) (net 3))
 (segment (start 132.3 96.9) (end 132 96.6) (width 0.4) (layer F.Cu) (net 3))
 (segment (start 133.2 96.9) (end 132.3 96.9) (width 0.4) (layer F.Cu) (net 3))
 (segment (start 132 96.6) (end 132 96.7) (width 0.4) (layer F.Cu) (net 3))
 (segment (start 132 97.2) (end 132.3 96.9) (width 0.4) (layer F.Cu) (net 3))
 (segment (start 132 96.7) (end 132 97.2) (width 0.4) (layer F.Cu) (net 3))
 (segment (start 132 97.2) (end 132 97.875) (width 0.4) (layer F.Cu) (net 3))
 (segment (start 132.075 97.025) (end 132.2 96.9) (width 0.4) (layer F.Cu) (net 3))
 (segment (start 132.075 97.95) (end 132.075 97.025) (width 0.4) (layer F.Cu) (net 3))
 (via (at 132 96.7) (size 0.8) (drill 0.4) (layers F.Cu B.Cu) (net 3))
 (segment (start 132.075 96.775) (end 132 96.7) (width 0.4) (layer F.Cu) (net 3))
 (segment (start 132.075 97.95) (end 132.075 96.775) (width 0.4) (layer F.Cu) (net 3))
 (segment (start 134.375 98.1) (end 132.3 98.1) (width 0.4) (layer B.Cu) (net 3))
 (segment (start 132 97.8) (end 132 96.7) (width 0.4) (layer B.Cu) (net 3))
 (segment (start 132.3 98.1) (end 132 97.8) (width 0.4) (layer B.Cu) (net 3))
 (via (at 137.9 96.5) (size 0.8) (drill 0.4) (layers F.Cu B.Cu) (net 1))
 (segment (start 137.9 97.975) (end 137.9 96.5) (width 0.4) (layer F.Cu) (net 1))
 (segment (start 137.9 96.5) (end 137.9 97.9) (width 0.4) (layer B.Cu) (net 1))
 (segment (start 137.7 98.1) (end 135.87501 98.1) (width 0.4) (layer B.Cu) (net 1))
 (segment (start 137.9 97.9) (end 137.7 98.1) (width 0.4) (layer B.Cu) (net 1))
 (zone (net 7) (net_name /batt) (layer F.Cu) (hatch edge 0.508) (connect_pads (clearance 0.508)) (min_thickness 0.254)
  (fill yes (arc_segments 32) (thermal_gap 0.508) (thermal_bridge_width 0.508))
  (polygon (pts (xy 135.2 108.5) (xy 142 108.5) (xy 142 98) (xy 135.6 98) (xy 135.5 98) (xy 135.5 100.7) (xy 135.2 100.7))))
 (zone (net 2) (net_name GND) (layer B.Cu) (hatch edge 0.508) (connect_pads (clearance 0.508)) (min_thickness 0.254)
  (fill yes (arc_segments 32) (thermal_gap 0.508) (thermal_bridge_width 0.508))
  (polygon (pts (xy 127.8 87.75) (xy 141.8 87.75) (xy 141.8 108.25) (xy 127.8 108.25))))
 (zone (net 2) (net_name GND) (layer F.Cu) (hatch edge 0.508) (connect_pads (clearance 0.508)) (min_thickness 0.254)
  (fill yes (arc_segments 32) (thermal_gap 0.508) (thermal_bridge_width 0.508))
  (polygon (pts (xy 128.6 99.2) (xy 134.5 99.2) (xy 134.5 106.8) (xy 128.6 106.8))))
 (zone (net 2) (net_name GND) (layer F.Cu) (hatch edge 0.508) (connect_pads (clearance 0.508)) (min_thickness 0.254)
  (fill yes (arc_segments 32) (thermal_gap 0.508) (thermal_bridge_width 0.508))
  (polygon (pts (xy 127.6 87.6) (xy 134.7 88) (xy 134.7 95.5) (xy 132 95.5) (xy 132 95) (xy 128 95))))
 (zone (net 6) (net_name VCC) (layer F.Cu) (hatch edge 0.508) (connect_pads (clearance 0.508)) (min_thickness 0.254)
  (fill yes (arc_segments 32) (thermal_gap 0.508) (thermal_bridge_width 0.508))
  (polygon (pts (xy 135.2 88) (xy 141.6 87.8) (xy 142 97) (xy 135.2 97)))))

